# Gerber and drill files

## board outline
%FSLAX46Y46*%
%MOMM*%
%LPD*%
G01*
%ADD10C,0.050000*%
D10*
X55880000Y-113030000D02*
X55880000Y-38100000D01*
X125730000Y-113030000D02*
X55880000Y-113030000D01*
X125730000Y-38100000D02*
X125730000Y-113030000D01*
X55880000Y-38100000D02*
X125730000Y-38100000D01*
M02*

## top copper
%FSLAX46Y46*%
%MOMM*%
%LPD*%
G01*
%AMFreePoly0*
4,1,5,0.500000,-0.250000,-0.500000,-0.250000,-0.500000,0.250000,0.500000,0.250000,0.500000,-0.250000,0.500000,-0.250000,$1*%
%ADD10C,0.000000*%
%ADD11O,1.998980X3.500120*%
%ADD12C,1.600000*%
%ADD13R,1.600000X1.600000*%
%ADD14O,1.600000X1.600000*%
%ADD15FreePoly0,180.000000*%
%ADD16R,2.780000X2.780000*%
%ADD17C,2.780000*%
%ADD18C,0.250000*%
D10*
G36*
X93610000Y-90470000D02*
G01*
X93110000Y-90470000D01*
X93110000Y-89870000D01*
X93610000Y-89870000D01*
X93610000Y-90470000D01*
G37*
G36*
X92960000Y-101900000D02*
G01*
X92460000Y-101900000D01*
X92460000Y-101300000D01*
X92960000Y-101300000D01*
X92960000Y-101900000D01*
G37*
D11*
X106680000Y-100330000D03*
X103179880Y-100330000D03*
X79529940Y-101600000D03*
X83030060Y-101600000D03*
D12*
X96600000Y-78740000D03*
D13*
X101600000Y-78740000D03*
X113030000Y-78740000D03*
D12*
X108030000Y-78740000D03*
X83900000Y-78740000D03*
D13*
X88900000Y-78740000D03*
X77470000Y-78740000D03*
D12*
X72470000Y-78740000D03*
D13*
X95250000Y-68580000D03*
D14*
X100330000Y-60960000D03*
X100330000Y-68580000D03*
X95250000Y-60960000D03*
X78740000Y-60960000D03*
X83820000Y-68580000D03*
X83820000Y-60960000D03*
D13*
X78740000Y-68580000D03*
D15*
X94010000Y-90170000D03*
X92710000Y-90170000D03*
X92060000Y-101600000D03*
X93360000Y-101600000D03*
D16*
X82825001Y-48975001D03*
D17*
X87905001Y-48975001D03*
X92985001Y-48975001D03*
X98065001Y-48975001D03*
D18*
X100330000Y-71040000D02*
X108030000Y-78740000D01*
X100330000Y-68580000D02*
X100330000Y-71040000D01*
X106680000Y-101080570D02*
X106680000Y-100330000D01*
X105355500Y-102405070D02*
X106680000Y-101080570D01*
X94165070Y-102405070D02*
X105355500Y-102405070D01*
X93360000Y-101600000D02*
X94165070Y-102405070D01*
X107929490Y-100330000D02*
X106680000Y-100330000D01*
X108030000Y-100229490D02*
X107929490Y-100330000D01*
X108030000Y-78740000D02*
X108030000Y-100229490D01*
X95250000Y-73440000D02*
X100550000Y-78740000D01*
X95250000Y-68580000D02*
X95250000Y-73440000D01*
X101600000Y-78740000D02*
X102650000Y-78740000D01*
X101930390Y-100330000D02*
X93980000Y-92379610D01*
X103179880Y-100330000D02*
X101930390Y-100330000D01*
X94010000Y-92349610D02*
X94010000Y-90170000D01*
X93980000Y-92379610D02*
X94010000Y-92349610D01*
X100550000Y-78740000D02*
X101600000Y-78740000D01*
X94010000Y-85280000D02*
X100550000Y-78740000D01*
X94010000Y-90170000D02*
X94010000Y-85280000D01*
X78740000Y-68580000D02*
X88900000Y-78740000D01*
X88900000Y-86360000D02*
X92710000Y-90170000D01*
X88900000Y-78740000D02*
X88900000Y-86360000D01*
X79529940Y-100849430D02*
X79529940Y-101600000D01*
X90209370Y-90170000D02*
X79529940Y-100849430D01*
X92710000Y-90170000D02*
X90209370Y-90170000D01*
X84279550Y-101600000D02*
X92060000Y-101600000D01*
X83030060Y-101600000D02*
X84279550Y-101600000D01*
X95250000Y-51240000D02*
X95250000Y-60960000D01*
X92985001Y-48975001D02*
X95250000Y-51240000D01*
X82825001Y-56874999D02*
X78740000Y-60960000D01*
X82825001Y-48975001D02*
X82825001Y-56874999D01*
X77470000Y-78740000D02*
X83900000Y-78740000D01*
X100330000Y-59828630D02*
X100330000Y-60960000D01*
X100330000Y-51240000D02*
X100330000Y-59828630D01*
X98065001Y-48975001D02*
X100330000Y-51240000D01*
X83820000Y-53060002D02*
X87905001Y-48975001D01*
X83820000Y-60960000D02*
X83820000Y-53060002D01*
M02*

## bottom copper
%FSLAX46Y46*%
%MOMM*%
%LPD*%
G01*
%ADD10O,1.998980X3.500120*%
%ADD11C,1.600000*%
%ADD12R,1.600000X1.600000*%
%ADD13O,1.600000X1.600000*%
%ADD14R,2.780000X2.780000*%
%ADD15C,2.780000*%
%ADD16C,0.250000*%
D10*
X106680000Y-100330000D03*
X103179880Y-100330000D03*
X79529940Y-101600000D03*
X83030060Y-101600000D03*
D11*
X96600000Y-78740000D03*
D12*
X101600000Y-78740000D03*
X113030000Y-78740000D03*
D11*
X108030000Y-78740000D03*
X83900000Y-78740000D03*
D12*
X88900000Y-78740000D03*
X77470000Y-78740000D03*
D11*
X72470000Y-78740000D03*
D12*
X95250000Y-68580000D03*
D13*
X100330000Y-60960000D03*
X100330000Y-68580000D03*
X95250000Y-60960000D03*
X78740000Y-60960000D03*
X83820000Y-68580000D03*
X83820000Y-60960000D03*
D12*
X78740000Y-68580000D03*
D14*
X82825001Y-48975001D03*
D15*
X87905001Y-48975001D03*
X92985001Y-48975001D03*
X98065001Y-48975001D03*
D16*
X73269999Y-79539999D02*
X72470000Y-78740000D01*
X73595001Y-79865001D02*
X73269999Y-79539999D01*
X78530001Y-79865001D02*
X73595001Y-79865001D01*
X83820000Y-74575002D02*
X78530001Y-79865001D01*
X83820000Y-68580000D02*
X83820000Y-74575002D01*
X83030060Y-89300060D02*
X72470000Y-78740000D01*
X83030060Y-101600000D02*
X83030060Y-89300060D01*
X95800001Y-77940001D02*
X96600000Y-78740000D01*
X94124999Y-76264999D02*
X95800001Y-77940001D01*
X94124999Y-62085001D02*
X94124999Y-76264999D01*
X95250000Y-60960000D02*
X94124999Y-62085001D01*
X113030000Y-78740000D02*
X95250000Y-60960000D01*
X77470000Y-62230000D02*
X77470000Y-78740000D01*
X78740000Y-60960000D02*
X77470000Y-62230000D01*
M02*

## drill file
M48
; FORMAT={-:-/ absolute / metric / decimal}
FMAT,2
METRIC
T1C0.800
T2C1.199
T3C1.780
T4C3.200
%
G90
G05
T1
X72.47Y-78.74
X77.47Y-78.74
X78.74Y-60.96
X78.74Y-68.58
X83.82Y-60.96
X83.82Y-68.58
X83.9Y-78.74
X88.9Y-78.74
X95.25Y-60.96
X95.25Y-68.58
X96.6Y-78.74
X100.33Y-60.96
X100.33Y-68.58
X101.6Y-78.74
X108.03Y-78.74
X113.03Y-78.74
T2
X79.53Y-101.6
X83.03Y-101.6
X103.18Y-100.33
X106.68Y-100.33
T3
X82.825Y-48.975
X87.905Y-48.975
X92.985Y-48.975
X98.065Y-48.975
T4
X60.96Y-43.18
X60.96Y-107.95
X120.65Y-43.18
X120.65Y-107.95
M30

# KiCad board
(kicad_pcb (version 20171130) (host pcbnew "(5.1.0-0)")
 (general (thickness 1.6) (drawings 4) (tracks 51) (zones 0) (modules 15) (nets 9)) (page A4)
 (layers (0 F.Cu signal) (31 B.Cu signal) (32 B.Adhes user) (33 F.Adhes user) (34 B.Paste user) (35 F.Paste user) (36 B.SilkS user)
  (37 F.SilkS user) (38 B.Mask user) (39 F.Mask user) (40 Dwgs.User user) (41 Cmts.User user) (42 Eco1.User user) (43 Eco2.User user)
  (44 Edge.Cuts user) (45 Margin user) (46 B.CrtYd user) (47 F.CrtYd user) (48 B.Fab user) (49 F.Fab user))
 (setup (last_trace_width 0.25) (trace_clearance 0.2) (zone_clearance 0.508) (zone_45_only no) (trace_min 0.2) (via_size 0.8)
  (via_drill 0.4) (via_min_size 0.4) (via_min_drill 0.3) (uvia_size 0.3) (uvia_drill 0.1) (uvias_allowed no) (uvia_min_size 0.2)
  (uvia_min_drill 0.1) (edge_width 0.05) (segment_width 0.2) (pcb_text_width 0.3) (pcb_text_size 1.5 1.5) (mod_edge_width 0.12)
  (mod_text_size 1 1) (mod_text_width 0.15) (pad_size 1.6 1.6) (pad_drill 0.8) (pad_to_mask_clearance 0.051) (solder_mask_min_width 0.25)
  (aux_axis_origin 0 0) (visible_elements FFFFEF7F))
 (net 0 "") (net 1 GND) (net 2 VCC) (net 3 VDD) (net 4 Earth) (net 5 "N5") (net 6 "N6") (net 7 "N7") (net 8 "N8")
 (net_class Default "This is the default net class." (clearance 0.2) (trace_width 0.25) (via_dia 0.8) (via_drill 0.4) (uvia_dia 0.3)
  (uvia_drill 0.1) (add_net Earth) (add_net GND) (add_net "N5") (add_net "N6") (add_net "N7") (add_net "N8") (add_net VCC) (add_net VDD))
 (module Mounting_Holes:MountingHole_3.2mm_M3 (layer F.Cu) (at 120.65 43.18)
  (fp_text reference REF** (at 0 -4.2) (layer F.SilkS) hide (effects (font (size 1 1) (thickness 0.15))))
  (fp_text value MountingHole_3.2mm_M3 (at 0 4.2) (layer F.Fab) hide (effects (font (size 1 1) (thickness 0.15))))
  (pad 1 np_thru_hole circle (at 0 0) (size 3.2 3.2) (drill 3.2) (layers *.Cu *.Mask)))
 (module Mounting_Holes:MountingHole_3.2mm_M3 (layer F.Cu) (at 120.65 107.95)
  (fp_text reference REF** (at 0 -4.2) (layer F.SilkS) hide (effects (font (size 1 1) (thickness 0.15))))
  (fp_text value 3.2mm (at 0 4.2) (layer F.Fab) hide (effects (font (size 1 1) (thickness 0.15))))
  (pad 1 np_thru_hole circle (at 0 0) (size 3.2 3.2) (drill 3.2) (layers *.Cu *.Mask)))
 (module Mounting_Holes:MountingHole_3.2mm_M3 (layer F.Cu) (at 60.96 107.95)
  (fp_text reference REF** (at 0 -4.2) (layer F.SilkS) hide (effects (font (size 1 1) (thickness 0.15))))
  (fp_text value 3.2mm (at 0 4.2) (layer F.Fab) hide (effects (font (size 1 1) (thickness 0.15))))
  (pad 1 np_thru_hole circle (at 0 0) (size 3.2 3.2) (drill 3.2) (layers *.Cu *.Mask)))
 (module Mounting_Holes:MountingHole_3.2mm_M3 (layer F.Cu) (at 60.96 43.18)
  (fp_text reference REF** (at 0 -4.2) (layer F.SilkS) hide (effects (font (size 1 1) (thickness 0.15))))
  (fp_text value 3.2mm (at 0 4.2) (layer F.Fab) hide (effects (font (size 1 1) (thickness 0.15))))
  (pad 1 np_thru_hole circle (at 0 0) (size 3.2 3.2) (drill 3.2) (layers *.Cu *.Mask)))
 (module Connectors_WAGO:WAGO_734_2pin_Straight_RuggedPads (layer F.Cu) (at 104.92994 100.33 180)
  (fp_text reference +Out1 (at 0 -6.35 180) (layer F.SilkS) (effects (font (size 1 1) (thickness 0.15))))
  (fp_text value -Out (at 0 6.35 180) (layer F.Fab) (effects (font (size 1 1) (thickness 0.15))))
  (pad 1 thru_hole oval (at -1.75006 0 180) (size 1.99898 3.50012) (drill 1.19888) (layers *.Cu *.Mask) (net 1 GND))
  (pad 2 thru_hole oval (at 1.75006 0 180) (size 1.99898 3.50012) (drill 1.19888) (layers *.Cu *.Mask) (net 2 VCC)))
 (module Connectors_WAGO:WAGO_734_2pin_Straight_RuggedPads (layer F.Cu) (at 81.28 101.6 180)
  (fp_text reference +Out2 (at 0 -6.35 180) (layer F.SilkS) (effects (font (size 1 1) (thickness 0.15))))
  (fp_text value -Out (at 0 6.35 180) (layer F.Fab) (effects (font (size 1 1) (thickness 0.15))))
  (pad 2 thru_hole oval (at 1.75006 0 180) (size 1.99898 3.50012) (drill 1.19888) (layers *.Cu *.Mask) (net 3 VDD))
  (pad 1 thru_hole oval (at -1.75006 0 180) (size 1.99898 3.50012) (drill 1.19888) (layers *.Cu *.Mask) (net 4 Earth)))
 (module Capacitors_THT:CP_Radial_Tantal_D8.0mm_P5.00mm (layer F.Cu) (at 101.6 78.74 180)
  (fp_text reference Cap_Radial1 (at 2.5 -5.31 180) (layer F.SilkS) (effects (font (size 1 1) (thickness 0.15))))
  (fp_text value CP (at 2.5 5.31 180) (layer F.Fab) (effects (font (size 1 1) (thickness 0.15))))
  (pad 2 thru_hole circle (at 5 0 180) (size 1.6 1.6) (drill 0.8) (layers *.Cu *.Mask) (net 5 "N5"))
  (pad 1 thru_hole rect (at 0 0 180) (size 1.6 1.6) (drill 0.8) (layers *.Cu *.Mask) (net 2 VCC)))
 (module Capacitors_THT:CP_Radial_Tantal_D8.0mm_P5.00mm (layer F.Cu) (at 113.03 78.74 180)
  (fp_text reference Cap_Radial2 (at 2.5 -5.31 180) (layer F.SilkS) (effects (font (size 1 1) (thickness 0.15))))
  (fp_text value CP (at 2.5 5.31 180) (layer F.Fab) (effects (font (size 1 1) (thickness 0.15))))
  (pad 1 thru_hole rect (at 0 0 180) (size 1.6 1.6) (drill 0.8) (layers *.Cu *.Mask) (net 5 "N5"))
  (pad 2 thru_hole circle (at 5 0 180) (size 1.6 1.6) (drill 0.8) (layers *.Cu *.Mask) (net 1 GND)))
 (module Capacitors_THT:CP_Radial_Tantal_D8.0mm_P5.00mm (layer F.Cu) (at 88.9 78.74 180)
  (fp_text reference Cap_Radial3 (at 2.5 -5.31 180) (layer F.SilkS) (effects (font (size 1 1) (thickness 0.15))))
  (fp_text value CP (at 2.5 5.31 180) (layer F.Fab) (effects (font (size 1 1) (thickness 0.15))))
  (pad 2 thru_hole circle (at 5 0 180) (size 1.6 1.6) (drill 0.8) (layers *.Cu *.Mask) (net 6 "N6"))
  (pad 1 thru_hole rect (at 0 0 180) (size 1.6 1.6) (drill 0.8) (layers *.Cu *.Mask) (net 3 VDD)))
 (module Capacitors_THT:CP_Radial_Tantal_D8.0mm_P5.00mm (layer F.Cu) (at 77.47 78.74 180)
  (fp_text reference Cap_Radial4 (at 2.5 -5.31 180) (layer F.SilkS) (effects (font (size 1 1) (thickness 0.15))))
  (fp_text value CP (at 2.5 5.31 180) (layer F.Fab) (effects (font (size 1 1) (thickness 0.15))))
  (pad 1 thru_hole rect (at 0 0 180) (size 1.6 1.6) (drill 0.8) (layers *.Cu *.Mask) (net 6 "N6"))
  (pad 2 thru_hole circle (at 5 0 180) (size 1.6 1.6) (drill 0.8) (layers *.Cu *.Mask) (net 4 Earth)))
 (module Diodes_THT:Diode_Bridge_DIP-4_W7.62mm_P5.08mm (layer F.Cu) (at 95.25 68.58 90)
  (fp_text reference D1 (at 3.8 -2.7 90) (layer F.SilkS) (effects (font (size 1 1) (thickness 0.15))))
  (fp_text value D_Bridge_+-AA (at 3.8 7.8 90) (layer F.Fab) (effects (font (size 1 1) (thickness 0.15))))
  (pad 1 thru_hole rect (at 0 0 90) (size 1.6 1.6) (drill 0.8) (layers *.Cu *.Mask) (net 2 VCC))
  (pad 3 thru_hole oval (at 7.62 5.08 90) (size 1.6 1.6) (drill 0.8) (layers *.Cu *.Mask) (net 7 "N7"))
  (pad 2 thru_hole oval (at 0 5.08 90) (size 1.6 1.6) (drill 0.8) (layers *.Cu *.Mask) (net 1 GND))
  (pad 4 thru_hole oval (at 7.62 0 90) (size 1.6 1.6) (drill 0.8) (layers *.Cu *.Mask) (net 5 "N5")))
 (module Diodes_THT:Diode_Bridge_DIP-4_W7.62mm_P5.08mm (layer F.Cu) (at 78.74 68.58 90)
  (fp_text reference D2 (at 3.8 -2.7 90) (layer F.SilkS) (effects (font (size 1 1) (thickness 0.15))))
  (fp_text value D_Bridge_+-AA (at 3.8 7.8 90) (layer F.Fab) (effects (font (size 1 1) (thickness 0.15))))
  (pad 4 thru_hole oval (at 7.62 0 90) (size 1.6 1.6) (drill 0.8) (layers *.Cu *.Mask) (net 6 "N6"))
  (pad 2 thru_hole oval (at 0 5.08 90) (size 1.6 1.6) (drill 0.8) (layers *.Cu *.Mask) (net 4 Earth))
  (pad 3 thru_hole oval (at 7.62 5.08 90) (size 1.6 1.6) (drill 0.8) (layers *.Cu *.Mask) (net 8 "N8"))
  (pad 1 thru_hole rect (at 0 0 90) (size 1.6 1.6) (drill 0.8) (layers *.Cu *.Mask) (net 3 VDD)))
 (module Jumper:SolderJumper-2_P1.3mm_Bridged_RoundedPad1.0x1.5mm (layer F.Cu) (at 93.36 90.17 180)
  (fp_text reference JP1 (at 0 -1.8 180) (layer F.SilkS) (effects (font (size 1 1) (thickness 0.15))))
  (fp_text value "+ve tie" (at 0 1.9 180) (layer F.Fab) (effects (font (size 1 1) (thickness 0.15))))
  (fp_poly (pts (xy 0.25 -0.3) (xy -0.25 -0.3) (xy -0.25 0.3) (xy 0.25 0.3)) (layer F.Cu) (width 0))
  (pad 1 smd custom (at -0.65 0 180) (size 1 0.5) (layers F.Cu F.Mask) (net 2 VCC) (zone_connect 2)
   (options (clearance outline) (anchor rect)) (primitives))
  (pad 2 smd custom (at 0.65 0 180) (size 1 0.5) (layers F.Cu F.Mask) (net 3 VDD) (zone_connect 2)
   (options (clearance outline) (anchor rect)) (primitives)))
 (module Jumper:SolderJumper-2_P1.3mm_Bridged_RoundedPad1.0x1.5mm (layer F.Cu) (at 92.71 101.6 180)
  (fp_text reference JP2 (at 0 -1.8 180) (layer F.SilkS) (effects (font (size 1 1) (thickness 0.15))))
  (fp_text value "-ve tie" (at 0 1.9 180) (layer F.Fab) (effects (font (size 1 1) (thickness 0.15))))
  (fp_poly (pts (xy 0.25 -0.3) (xy -0.25 -0.3) (xy -0.25 0.3) (xy 0.25 0.3)) (layer F.Cu) (width 0))
  (pad 2 smd custom (at 0.65 0 180) (size 1 0.5) (layers F.Cu F.Mask) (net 4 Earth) (zone_connect 2)
   (options (clearance outline) (anchor rect)) (primitives))
  (pad 1 smd custom (at -0.65 0 180) (size 1 0.5) (layers F.Cu F.Mask) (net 1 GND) (zone_connect 2)
   (options (clearance outline) (anchor rect)) (primitives)))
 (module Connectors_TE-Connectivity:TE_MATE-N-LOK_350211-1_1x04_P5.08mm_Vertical (layer F.Cu) (at 82.825001 48.975001)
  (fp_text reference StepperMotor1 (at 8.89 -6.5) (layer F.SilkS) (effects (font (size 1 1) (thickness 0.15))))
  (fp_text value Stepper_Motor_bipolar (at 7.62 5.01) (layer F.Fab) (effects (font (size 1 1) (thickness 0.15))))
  (pad 1 thru_hole rect (at 0 0) (size 2.78 2.78) (drill 1.78) (layers *.Cu *.Mask) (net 6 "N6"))
  (pad 2 thru_hole circle (at 5.08 0) (size 2.78 2.78) (drill 1.78) (layers *.Cu *.Mask) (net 8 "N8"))
  (pad 3 thru_hole circle (at 10.16 0) (size 2.78 2.78) (drill 1.78) (layers *.Cu *.Mask) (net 5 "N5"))
  (pad 4 thru_hole circle (at 15.24 0) (size 2.78 2.78) (drill 1.78) (layers *.Cu *.Mask) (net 7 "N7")))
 (gr_line (start 55.88 113.03) (end 55.88 38.1) (layer Edge.Cuts) (width 0.05))
 (gr_line (start 125.73 113.03) (end 55.88 113.03) (layer Edge.Cuts) (width 0.05))
 (gr_line (start 125.73 38.1) (end 125.73 113.03) (layer Edge.Cuts) (width 0.05))
 (gr_line (start 55.88 38.1) (end 125.73 38.1) (layer Edge.Cuts) (width 0.05))
 (segment (start 100.33 71.04) (end 108.03 78.74) (width 0.25) (layer F.Cu) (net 1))
 (segment (start 100.33 68.58) (end 100.33 71.04) (width 0.25) (layer F.Cu) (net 1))
 (segment (start 106.68 101.08057) (end 106.68 100.33) (width 0.25) (layer F.Cu) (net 1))
 (segment (start 105.3555 102.40507) (end 106.68 101.08057) (width 0.25) (layer F.Cu) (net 1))
 (segment (start 94.16507 102.40507) (end 105.3555 102.40507) (width 0.25) (layer F.Cu) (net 1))
 (segment (start 93.36 101.6) (end 94.16507 102.40507) (width 0.25) (layer F.Cu) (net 1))
 (segment (start 107.92949 100.33) (end 106.68 100.33) (width 0.25) (layer F.Cu) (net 1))
 (segment (start 108.03 100.22949) (end 107.92949 100.33) (width 0.25) (layer F.Cu) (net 1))
 (segment (start 108.03 78.74) (end 108.03 100.22949) (width 0.25) (layer F.Cu) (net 1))
 (segment (start 95.25 73.44) (end 100.55 78.74) (width 0.25) (layer F.Cu) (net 2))
 (segment (start 95.25 68.58) (end 95.25 73.44) (width 0.25) (layer F.Cu) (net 2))
 (segment (start 101.6 78.74) (end 102.65 78.74) (width 0.25) (layer F.Cu) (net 2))
 (segment (start 101.93039 100.33) (end 93.98 92.37961) (width 0.25) (layer F.Cu) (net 2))
 (segment (start 103.17988 100.33) (end 101.93039 100.33) (width 0.25) (layer F.Cu) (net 2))
 (segment (start 94.01 92.34961) (end 94.01 90.17) (width 0.25) (layer F.Cu) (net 2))
 (segment (start 93.98 92.37961) (end 94.01 92.34961) (width 0.25) (layer F.Cu) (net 2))
 (segment (start 100.55 78.74) (end 101.6 78.74) (width 0.25) (layer F.Cu) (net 2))
 (segment (start 94.01 85.28) (end 100.55 78.74) (width 0.25) (layer F.Cu) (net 2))
 (segment (start 94.01 90.17) (end 94.01 85.28) (width 0.25) (layer F.Cu) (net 2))
 (segment (start 78.74 68.58) (end 88.9 78.74) (width 0.25) (layer F.Cu) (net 3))
 (segment (start 88.9 86.36) (end 92.71 90.17) (width 0.25) (layer F.Cu) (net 3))
 (segment (start 88.9 78.74) (end 88.9 86.36) (width 0.25) (layer F.Cu) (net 3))
 (segment (start 79.52994 100.84943) (end 79.52994 101.6) (width 0.25) (layer F.Cu) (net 3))
 (segment (start 90.20937 90.17) (end 79.52994 100.84943) (width 0.25) (layer F.Cu) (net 3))
 (segment (start 92.71 90.17) (end 90.20937 90.17) (width 0.25) (layer F.Cu) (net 3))
 (segment (start 73.269999 79.539999) (end 72.47 78.74) (width 0.25) (layer B.Cu) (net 4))
 (segment (start 73.595001 79.865001) (end 73.269999 79.539999) (width 0.25) (layer B.Cu) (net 4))
 (segment (start 78.530001 79.865001) (end 73.595001 79.865001) (width 0.25) (layer B.Cu) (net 4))
 (segment (start 83.82 74.575002) (end 78.530001 79.865001) (width 0.25) (layer B.Cu) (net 4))
 (segment (start 83.82 68.58) (end 83.82 74.575002) (width 0.25) (layer B.Cu) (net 4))
 (segment (start 84.27955 101.6) (end 92.06 101.6) (width 0.25) (layer F.Cu) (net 4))
 (segment (start 83.03006 101.6) (end 84.27955 101.6) (width 0.25) (layer F.Cu) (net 4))
 (segment (start 83.03006 89.30006) (end 72.47 78.74) (width 0.25) (layer B.Cu) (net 4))
 (segment (start 83.03006 101.6) (end 83.03006 89.30006) (width 0.25) (layer B.Cu) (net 4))
 (segment (start 95.25 51.24) (end 95.25 60.96) (width 0.25) (layer F.Cu) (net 5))
 (segment (start 92.985001 48.975001) (end 95.25 51.24) (width 0.25) (layer F.Cu) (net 5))
 (segment (start 95.800001 77.940001) (end 96.6 78.74) (width 0.25) (layer B.Cu) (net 5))
 (segment (start 94.124999 76.264999) (end 95.800001 77.940001) (width 0.25) (layer B.Cu) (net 5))
 (segment (start 94.124999 62.085001) (end 94.124999 76.264999) (width 0.25) (layer B.Cu) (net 5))
 (segment (start 95.25 60.96) (end 94.124999 62.085001) (width 0.25) (layer B.Cu) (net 5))
 (segment (start 113.03 78.74) (end 95.25 60.96) (width 0.25) (layer B.Cu) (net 5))
 (segment (start 82.825001 56.874999) (end 78.74 60.96) (width 0.25) (layer F.Cu) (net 6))
 (segment (start 82.825001 48.975001) (end 82.825001 56.874999) (width 0.25) (layer F.Cu) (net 6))
 (segment (start 77.47 62.23) (end 77.47 78.74) (width 0.25) (layer B.Cu) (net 6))
 (segment (start 78.74 60.96) (end 77.47 62.23) (width 0.25) (layer B.Cu) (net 6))
 (segment (start 77.47 78.74) (end 83.9 78.74) (width 0.25) (layer F.Cu) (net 6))
 (segment (start 100.33 59.82863) (end 100.33 60.96) (width 0.25) (layer F.Cu) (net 7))
 (segment (start 100.33 51.24) (end 100.33 59.82863) (width 0.25) (layer F.Cu) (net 7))
 (segment (start 98.065001 48.975001) (end 100.33 51.24) (width 0.25) (layer F.Cu) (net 7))
 (segment (start 83.82 53.060002) (end 87.905001 48.975001) (width 0.25) (layer F.Cu) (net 8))
 (segment (start 83.82 60.96) (end 83.82 53.060002) (width 0.25) (layer F.Cu) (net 8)))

